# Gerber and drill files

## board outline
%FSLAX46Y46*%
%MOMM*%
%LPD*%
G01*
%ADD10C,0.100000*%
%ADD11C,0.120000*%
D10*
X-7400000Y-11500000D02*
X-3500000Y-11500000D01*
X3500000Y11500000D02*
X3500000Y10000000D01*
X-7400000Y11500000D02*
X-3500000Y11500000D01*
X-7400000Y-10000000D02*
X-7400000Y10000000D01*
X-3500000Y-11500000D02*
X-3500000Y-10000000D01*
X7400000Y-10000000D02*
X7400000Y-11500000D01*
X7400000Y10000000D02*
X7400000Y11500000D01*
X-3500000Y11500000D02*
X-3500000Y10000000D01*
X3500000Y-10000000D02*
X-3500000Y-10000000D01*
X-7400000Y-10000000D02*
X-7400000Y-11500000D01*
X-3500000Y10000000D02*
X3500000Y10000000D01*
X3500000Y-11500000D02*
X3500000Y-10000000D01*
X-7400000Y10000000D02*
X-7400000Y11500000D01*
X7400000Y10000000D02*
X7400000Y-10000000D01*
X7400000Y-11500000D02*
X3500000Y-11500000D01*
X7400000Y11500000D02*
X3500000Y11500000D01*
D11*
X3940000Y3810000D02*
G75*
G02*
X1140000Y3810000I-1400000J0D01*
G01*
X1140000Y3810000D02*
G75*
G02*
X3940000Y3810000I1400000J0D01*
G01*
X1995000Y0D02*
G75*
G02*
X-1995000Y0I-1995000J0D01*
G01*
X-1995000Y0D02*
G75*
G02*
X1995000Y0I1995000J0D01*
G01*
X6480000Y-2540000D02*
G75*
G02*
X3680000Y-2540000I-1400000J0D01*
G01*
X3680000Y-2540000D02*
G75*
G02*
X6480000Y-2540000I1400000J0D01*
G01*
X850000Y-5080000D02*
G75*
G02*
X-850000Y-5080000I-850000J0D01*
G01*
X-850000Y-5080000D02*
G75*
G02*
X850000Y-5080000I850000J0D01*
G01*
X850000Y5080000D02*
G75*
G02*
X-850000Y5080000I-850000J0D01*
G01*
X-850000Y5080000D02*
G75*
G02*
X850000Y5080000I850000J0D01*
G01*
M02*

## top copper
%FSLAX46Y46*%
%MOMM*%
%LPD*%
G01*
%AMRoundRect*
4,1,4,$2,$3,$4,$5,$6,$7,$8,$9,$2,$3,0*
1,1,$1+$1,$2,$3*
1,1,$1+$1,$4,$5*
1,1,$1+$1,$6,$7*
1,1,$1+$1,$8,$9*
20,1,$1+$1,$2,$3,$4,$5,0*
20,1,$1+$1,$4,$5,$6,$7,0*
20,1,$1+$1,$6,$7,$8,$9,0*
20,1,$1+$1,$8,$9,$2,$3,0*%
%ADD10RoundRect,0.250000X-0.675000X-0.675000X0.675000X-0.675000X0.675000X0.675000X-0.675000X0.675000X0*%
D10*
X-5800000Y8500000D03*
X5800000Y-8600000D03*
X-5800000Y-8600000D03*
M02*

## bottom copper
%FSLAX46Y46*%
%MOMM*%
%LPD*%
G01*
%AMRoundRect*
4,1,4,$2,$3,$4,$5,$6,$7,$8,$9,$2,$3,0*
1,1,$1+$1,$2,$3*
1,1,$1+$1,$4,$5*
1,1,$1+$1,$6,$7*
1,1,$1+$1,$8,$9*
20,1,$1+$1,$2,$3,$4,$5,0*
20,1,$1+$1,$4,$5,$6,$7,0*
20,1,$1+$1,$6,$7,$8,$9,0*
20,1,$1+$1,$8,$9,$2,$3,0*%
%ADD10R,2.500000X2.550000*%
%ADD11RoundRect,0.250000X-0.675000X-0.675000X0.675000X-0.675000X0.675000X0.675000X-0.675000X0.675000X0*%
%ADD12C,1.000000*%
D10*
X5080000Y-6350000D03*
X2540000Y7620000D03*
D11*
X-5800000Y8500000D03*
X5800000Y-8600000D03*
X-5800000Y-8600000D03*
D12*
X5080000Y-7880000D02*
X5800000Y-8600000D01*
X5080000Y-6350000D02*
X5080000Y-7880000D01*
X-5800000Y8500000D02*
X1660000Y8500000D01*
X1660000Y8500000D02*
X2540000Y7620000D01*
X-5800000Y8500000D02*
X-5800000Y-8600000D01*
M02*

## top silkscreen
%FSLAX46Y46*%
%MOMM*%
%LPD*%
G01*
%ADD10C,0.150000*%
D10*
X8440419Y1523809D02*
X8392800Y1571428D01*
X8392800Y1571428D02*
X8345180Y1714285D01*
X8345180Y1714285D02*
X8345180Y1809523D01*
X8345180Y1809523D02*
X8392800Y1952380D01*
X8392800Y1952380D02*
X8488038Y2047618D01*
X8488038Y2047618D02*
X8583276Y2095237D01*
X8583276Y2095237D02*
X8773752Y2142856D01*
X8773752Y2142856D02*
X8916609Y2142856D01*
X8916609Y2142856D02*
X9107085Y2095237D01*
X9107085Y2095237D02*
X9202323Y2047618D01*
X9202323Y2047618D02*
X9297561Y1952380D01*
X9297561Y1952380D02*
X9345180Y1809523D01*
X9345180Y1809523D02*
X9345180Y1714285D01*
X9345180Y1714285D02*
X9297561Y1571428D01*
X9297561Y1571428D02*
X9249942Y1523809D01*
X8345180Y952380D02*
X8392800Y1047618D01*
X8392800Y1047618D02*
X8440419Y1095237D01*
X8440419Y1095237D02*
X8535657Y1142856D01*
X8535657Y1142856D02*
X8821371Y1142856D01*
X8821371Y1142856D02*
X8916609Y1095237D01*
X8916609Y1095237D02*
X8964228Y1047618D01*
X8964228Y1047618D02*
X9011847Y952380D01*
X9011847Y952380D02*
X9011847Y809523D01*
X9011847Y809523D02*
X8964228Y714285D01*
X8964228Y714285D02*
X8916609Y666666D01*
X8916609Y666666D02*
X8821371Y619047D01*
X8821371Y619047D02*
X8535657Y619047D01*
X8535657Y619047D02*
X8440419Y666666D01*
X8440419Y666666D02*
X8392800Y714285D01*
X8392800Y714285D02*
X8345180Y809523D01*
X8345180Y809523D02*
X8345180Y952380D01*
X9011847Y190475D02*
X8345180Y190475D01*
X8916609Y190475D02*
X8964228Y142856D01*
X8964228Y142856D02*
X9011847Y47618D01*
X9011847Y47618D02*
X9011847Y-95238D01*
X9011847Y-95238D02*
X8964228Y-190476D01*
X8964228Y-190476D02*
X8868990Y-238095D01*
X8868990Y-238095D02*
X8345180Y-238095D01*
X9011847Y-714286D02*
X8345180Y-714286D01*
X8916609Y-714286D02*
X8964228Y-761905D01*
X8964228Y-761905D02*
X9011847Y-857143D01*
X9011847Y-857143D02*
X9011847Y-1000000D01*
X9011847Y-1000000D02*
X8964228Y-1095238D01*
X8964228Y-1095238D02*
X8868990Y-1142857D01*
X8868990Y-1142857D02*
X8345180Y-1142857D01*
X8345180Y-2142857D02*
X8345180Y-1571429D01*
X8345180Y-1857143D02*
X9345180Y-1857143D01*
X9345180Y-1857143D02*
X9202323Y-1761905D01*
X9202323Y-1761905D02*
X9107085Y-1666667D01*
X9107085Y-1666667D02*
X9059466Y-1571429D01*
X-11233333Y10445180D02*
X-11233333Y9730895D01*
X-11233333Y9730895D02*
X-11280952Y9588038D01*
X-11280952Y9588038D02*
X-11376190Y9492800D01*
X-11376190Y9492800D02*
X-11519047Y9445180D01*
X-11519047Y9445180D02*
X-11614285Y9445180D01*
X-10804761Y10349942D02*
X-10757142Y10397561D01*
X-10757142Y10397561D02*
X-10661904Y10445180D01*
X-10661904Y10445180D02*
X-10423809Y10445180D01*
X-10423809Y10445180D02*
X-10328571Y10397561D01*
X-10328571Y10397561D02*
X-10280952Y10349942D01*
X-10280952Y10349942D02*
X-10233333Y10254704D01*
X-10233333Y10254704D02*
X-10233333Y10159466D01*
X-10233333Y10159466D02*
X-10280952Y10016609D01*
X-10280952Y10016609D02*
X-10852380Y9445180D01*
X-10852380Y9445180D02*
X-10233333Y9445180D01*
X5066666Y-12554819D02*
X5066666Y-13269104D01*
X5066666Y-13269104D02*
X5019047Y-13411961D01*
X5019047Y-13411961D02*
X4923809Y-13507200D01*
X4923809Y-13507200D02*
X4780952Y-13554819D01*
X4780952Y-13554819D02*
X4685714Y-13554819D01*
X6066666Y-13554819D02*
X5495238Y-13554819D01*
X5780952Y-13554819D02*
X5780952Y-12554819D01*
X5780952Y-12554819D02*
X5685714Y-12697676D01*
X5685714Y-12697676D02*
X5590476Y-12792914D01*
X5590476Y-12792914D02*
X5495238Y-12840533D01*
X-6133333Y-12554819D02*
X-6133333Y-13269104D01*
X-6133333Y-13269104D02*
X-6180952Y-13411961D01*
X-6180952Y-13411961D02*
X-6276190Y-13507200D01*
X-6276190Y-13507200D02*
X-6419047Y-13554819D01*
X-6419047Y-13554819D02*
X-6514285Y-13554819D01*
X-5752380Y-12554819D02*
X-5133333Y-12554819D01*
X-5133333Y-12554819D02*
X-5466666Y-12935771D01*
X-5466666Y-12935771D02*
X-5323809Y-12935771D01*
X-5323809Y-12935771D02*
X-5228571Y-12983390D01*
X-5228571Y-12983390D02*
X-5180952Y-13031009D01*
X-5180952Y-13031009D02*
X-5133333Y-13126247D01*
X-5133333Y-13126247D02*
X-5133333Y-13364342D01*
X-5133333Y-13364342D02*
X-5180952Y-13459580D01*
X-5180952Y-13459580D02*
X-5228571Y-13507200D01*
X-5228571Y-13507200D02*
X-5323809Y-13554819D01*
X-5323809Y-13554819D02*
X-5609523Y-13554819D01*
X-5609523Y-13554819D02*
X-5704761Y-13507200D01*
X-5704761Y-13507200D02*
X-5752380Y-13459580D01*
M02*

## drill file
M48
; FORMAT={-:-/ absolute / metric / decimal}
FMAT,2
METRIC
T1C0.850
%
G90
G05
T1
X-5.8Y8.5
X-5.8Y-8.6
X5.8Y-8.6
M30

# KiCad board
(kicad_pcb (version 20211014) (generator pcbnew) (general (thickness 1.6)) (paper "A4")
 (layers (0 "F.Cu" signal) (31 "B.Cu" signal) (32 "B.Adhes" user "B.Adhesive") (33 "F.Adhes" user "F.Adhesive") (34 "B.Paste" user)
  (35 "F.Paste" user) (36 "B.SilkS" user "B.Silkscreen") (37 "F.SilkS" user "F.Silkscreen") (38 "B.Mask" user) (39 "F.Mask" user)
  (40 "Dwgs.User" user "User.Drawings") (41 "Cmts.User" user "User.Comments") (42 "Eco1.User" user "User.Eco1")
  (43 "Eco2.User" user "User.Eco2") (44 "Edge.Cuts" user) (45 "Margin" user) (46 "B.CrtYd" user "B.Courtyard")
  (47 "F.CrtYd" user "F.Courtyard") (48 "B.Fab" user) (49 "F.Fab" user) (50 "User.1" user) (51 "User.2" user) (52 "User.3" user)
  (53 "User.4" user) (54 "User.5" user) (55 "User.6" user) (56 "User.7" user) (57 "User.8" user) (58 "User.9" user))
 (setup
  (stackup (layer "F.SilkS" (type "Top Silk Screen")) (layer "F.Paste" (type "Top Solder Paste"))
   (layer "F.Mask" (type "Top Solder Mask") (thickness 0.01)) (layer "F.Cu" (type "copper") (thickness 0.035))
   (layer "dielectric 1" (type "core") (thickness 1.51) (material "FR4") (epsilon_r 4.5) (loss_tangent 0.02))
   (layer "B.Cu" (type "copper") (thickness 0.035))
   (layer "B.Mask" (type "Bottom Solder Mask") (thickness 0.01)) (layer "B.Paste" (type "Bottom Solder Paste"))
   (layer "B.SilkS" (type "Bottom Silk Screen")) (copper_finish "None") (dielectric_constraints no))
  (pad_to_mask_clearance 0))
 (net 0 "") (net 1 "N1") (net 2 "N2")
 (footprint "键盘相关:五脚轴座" (layer "F.Cu") (at 0 0 -90)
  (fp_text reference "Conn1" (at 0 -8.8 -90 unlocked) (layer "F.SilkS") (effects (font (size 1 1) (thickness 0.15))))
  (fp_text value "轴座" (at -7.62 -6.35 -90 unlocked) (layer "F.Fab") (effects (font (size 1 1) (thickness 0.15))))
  (fp_circle (center -3.81 -2.54) (end -2.41 -2.54) (layer "Edge.Cuts") (width 0.12) (fill none))
  (fp_circle (center 0 0) (end 1.995 0) (layer "Edge.Cuts") (width 0.12) (fill none))
  (fp_circle (center 2.54 -5.08) (end 3.94 -5.08) (layer "Edge.Cuts") (width 0.12) (fill none))
  (fp_circle (center 5.08 0) (end 5.93 0) (layer "Edge.Cuts") (width 0.12) (fill none))
  (fp_circle (center -5.08 0) (end -4.23 0) (layer "Edge.Cuts") (width 0.12) (fill none))
  (pad "1" smd rect (at 6.35 -5.08 270) (size 2.55 2.5) (layers "B.Cu" "B.Paste" "B.Mask") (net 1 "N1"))
  (pad "2" smd rect (at -7.62 -2.54 270) (size 2.55 2.5) (layers "B.Cu" "B.Paste" "B.Mask") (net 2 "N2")))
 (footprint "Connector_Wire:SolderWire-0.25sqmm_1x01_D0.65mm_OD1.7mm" (layer "F.Cu") (at -5.8 -8.6)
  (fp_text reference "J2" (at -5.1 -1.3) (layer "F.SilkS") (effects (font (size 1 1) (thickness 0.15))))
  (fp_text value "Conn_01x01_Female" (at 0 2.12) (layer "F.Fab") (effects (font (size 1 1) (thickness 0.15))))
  (pad "1" thru_hole roundrect (at 0 0.1) (size 1.85 1.85) (drill 0.85) (layers *.Cu *.Mask) (roundrect_rratio 0.135135) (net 2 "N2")))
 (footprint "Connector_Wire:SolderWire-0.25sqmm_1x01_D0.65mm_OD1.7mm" (layer "F.Cu") (at 5.8 8.6)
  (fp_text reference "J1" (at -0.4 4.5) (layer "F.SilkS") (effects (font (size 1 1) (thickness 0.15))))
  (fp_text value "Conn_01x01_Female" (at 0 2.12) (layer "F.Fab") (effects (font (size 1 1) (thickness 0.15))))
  (pad "1" thru_hole roundrect (at 0 0) (size 1.85 1.85) (drill 0.85) (layers *.Cu *.Mask) (roundrect_rratio 0.135135) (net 1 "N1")))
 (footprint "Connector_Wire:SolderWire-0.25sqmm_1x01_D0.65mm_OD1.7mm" (layer "F.Cu") (at -5.8 8.6)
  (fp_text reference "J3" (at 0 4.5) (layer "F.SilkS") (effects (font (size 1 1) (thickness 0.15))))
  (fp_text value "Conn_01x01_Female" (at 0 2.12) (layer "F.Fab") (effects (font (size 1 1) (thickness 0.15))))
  (pad "1" thru_hole roundrect (at 0 0) (size 1.85 1.85) (drill 0.85) (layers *.Cu *.Mask) (roundrect_rratio 0.135135) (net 2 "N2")))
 (gr_line (start -7.4 11.5) (end -3.5 11.5) (layer "Edge.Cuts") (width 0.1))
 (gr_line (start 3.5 -11.5) (end 3.5 -10) (layer "Edge.Cuts") (width 0.1))
 (gr_line (start -7.4 -11.5) (end -3.5 -11.5) (layer "Edge.Cuts") (width 0.1))
 (gr_line (start -7.4 10) (end -7.4 -10) (layer "Edge.Cuts") (width 0.1))
 (gr_line (start -3.5 11.5) (end -3.5 10) (layer "Edge.Cuts") (width 0.1))
 (gr_line (start 7.4 10) (end 7.4 11.5) (layer "Edge.Cuts") (width 0.1))
 (gr_line (start 7.4 -10) (end 7.4 -11.5) (layer "Edge.Cuts") (width 0.1))
 (gr_line (start -3.5 -11.5) (end -3.5 -10) (layer "Edge.Cuts") (width 0.1))
 (gr_line (start 3.5 10) (end -3.5 10) (layer "Edge.Cuts") (width 0.1))
 (gr_line (start -7.4 10) (end -7.4 11.5) (layer "Edge.Cuts") (width 0.1))
 (gr_line (start -3.5 -10) (end 3.5 -10) (layer "Edge.Cuts") (width 0.1))
 (gr_line (start 3.5 11.5) (end 3.5 10) (layer "Edge.Cuts") (width 0.1))
 (gr_line (start -7.4 -10) (end -7.4 -11.5) (layer "Edge.Cuts") (width 0.1))
 (gr_line (start 7.4 -10) (end 7.4 10) (layer "Edge.Cuts") (width 0.1))
 (gr_line (start 7.4 11.5) (end 3.5 11.5) (layer "Edge.Cuts") (width 0.1))
 (gr_line (start 7.4 -11.5) (end 3.5 -11.5) (layer "Edge.Cuts") (width 0.1))
 (segment (start 5.08 7.88) (end 5.8 8.6) (width 1) (layer "B.Cu") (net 1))
 (segment (start 5.08 6.35) (end 5.08 7.88) (width 1) (layer "B.Cu") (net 1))
 (segment (start -5.8 -8.5) (end 1.66 -8.5) (width 1) (layer "B.Cu") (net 2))
 (segment (start 1.66 -8.5) (end 2.54 -7.62) (width 1) (layer "B.Cu") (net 2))
 (segment (start -5.8 -8.5) (end -5.8 8.6) (width 1) (layer "B.Cu") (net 2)))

